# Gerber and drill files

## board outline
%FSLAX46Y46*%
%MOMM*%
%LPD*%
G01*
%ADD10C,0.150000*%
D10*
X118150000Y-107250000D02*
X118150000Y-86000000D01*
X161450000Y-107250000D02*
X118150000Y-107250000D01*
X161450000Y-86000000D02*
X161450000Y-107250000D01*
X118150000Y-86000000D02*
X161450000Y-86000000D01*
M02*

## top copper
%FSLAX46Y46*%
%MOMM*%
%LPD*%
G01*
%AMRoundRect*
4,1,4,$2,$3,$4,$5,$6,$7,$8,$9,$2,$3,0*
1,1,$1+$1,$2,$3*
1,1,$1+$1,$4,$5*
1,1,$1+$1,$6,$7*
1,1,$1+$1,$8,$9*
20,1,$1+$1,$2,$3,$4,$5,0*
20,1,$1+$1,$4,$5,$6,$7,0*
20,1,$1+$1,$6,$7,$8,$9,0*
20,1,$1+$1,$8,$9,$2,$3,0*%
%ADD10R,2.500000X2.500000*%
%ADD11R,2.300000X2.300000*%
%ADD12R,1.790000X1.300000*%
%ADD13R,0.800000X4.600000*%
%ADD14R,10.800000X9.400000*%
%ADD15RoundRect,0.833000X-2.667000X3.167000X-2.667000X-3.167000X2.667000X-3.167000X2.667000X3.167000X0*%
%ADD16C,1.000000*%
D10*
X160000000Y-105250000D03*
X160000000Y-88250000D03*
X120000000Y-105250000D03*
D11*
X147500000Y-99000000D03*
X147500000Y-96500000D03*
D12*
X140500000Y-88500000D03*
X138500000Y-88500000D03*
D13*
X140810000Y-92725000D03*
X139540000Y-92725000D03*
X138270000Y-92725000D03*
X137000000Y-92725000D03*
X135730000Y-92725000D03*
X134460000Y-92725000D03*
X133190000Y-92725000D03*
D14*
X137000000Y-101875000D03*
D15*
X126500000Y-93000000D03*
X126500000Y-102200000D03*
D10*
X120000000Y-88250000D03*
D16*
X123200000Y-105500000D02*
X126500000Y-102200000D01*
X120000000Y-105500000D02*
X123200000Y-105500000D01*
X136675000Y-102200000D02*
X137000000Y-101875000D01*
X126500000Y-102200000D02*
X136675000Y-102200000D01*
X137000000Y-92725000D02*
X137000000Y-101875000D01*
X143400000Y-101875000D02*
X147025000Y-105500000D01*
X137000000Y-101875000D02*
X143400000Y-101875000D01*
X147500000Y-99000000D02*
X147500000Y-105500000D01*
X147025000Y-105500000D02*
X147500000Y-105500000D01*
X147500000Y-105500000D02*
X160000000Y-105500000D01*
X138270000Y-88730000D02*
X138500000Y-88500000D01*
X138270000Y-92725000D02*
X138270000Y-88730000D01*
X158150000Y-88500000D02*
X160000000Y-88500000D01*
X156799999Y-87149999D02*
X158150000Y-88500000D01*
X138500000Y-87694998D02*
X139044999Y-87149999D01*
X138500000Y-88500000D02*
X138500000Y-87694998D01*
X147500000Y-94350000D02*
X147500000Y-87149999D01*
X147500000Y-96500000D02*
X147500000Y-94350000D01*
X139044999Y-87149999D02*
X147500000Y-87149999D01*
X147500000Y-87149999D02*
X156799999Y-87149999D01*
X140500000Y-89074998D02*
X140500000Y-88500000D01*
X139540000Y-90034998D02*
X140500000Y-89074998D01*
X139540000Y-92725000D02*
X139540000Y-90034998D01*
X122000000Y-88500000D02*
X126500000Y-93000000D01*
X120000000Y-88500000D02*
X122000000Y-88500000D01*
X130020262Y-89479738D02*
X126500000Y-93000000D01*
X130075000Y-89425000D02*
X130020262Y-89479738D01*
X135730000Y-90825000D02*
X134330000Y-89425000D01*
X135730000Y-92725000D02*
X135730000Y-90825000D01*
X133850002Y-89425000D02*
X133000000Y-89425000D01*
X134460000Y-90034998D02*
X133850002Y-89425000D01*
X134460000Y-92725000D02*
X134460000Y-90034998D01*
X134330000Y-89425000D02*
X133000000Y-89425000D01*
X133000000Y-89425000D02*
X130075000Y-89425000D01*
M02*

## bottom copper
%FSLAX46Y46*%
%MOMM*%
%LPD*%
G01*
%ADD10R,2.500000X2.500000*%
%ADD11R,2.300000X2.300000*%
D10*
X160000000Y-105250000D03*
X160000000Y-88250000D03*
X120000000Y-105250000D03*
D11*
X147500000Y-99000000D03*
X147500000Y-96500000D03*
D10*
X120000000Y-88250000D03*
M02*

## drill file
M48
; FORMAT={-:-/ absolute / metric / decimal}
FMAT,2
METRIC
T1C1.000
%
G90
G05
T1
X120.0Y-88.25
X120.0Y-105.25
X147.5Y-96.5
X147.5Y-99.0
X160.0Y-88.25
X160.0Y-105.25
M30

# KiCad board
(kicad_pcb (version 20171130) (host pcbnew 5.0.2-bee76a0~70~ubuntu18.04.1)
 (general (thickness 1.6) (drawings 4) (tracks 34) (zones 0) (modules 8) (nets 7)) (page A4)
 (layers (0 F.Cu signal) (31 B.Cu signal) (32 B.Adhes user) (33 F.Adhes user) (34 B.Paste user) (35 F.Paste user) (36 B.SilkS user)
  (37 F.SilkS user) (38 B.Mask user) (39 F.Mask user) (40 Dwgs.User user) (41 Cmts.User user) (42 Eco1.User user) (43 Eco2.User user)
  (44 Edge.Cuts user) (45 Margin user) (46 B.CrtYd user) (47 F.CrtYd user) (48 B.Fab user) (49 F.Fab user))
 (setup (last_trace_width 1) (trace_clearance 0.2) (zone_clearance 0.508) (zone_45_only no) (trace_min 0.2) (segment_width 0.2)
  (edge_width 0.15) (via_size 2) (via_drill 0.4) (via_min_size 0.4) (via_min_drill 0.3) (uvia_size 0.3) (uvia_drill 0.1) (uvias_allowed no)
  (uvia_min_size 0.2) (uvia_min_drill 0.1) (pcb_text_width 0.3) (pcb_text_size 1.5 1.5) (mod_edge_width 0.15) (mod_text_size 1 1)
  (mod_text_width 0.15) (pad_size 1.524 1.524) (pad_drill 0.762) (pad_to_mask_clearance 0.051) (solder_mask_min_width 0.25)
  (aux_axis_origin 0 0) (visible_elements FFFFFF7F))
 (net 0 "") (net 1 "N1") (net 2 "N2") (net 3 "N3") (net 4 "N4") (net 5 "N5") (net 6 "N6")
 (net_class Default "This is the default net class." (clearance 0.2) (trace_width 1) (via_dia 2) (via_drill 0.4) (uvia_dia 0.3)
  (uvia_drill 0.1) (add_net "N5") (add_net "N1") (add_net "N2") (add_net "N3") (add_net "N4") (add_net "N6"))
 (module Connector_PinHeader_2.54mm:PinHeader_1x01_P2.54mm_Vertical (layer F.Cu) (at 160 105.25)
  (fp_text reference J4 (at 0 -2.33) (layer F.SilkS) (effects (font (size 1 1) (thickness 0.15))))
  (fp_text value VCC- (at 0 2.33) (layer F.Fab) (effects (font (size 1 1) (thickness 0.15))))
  (pad 1 thru_hole rect (at 0 0) (size 2.5 2.5) (drill 1) (layers *.Cu *.Mask) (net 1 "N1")))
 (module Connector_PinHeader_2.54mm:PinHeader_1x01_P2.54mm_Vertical (layer F.Cu) (at 160 88.25)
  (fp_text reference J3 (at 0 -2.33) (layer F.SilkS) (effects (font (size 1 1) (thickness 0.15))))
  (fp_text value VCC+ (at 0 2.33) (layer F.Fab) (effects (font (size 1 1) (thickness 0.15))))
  (pad 1 thru_hole rect (at 0 0) (size 2.5 2.5) (drill 1) (layers *.Cu *.Mask) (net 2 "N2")))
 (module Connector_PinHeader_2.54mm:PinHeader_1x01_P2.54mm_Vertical (layer F.Cu) (at 120 105.25)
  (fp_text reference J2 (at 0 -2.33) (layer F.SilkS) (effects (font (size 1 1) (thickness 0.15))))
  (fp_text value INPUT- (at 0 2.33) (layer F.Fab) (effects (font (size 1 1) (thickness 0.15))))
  (pad 1 thru_hole rect (at 0 0) (size 2.5 2.5) (drill 1) (layers *.Cu *.Mask) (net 1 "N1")))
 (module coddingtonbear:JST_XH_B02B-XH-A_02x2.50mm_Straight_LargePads (layer F.Cu) (at 147.5 96.5 270)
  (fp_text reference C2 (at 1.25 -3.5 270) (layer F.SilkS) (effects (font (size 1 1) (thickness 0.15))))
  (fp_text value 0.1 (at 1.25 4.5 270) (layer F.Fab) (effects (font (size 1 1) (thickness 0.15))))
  (pad 2 thru_hole rect (at 2.5 0 270) (size 2.3 2.3) (drill 1) (layers *.Cu *.Mask) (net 1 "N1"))
  (pad 1 thru_hole rect (at 0 0 270) (size 2.3 2.3) (drill 1) (layers *.Cu *.Mask) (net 2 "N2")))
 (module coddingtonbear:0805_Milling (layer F.Cu) (at 139.5 88.5)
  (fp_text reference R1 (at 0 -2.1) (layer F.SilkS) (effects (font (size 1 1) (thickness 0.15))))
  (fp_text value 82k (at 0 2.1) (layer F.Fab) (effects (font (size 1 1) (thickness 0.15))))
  (pad 2 smd rect (at 1 0) (size 1.79 1.3) (layers F.Cu F.Paste F.Mask) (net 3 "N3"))
  (pad 1 smd rect (at -1 0) (size 1.79 1.3) (layers F.Cu F.Paste F.Mask) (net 2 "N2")))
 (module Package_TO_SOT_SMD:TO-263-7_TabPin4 (layer F.Cu) (at 137 98.5 270)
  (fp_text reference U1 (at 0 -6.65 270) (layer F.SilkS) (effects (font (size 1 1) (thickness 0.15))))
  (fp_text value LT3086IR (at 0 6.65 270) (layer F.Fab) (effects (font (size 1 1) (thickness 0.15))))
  (pad 1 smd rect (at -5.775 -3.81 270) (size 4.6 0.8) (layers F.Cu F.Paste F.Mask) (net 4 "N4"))
  (pad 2 smd rect (at -5.775 -2.54 270) (size 4.6 0.8) (layers F.Cu F.Paste F.Mask) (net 3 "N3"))
  (pad 3 smd rect (at -5.775 -1.27 270) (size 4.6 0.8) (layers F.Cu F.Paste F.Mask) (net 2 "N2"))
  (pad 4 smd rect (at -5.775 0 270) (size 4.6 0.8) (layers F.Cu F.Paste F.Mask) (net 1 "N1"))
  (pad 5 smd rect (at -5.775 1.27 270) (size 4.6 0.8) (layers F.Cu F.Paste F.Mask) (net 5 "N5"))
  (pad 6 smd rect (at -5.775 2.54 270) (size 4.6 0.8) (layers F.Cu F.Paste F.Mask) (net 5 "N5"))
  (pad 7 smd rect (at -5.775 3.81 270) (size 4.6 0.8) (layers F.Cu F.Paste F.Mask) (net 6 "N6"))
  (pad 4 smd rect (at 3.375 0 270) (size 9.4 10.8) (layers F.Cu F.Mask) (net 1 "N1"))
  (pad "" smd rect (at 5.8 2.775 270) (size 4.55 5.25) (layers F.Paste))
  (pad "" smd rect (at 0.95 -2.775 270) (size 4.55 5.25) (layers F.Paste))
  (pad "" smd rect (at 5.8 -2.775 270) (size 4.55 5.25) (layers F.Paste))
  (pad "" smd rect (at 0.95 2.775 270) (size 4.55 5.25) (layers F.Paste)))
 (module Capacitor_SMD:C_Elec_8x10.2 (layer F.Cu) (at 126.5 97.6 270)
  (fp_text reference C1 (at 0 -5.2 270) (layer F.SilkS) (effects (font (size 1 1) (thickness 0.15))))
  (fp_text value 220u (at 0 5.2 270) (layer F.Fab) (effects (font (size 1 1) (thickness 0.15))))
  (pad 1 smd roundrect (at -4.6 0 270) (size 8 7) (layers F.Cu F.Paste F.Mask) (roundrect_rratio 0.119) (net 5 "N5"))
  (pad 2 smd roundrect (at 4.6 0 270) (size 8 7) (layers F.Cu F.Paste F.Mask) (roundrect_rratio 0.119) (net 1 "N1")))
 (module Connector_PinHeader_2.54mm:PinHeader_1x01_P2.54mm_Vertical (layer F.Cu) (at 120 88.25)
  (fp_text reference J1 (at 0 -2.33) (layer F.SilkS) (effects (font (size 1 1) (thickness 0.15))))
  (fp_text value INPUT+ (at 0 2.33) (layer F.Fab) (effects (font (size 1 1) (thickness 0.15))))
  (pad 1 thru_hole rect (at 0 0) (size 2.5 2.5) (drill 1) (layers *.Cu *.Mask) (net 5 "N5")))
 (gr_line (start 118.15 107.25) (end 118.15 86) (layer Edge.Cuts) (width 0.15))
 (gr_line (start 161.45 107.25) (end 118.15 107.25) (layer Edge.Cuts) (width 0.15))
 (gr_line (start 161.45 86) (end 161.45 107.25) (layer Edge.Cuts) (width 0.15))
 (gr_line (start 118.15 86) (end 161.45 86) (layer Edge.Cuts) (width 0.15))
 (segment (start 123.2 105.5) (end 126.5 102.2) (width 1) (layer F.Cu) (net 1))
 (segment (start 120 105.5) (end 123.2 105.5) (width 1) (layer F.Cu) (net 1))
 (segment (start 136.675 102.2) (end 137 101.875) (width 1) (layer F.Cu) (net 1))
 (segment (start 126.5 102.2) (end 136.675 102.2) (width 1) (layer F.Cu) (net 1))
 (segment (start 137 92.725) (end 137 101.875) (width 1) (layer F.Cu) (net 1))
 (segment (start 143.4 101.875) (end 147.025 105.5) (width 1) (layer F.Cu) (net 1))
 (segment (start 137 101.875) (end 143.4 101.875) (width 1) (layer F.Cu) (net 1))
 (segment (start 147.5 99) (end 147.5 105.5) (width 1) (layer F.Cu) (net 1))
 (segment (start 147.025 105.5) (end 147.5 105.5) (width 1) (layer F.Cu) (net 1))
 (segment (start 147.5 105.5) (end 160 105.5) (width 1) (layer F.Cu) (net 1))
 (segment (start 138.27 88.73) (end 138.5 88.5) (width 1) (layer F.Cu) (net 2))
 (segment (start 138.27 92.725) (end 138.27 88.73) (width 1) (layer F.Cu) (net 2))
 (segment (start 158.15 88.5) (end 160 88.5) (width 1) (layer F.Cu) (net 2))
 (segment (start 156.799999 87.149999) (end 158.15 88.5) (width 1) (layer F.Cu) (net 2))
 (segment (start 138.5 87.694998) (end 139.044999 87.149999) (width 1) (layer F.Cu) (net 2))
 (segment (start 138.5 88.5) (end 138.5 87.694998) (width 1) (layer F.Cu) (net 2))
 (segment (start 147.5 94.35) (end 147.5 87.149999) (width 1) (layer F.Cu) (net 2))
 (segment (start 147.5 96.5) (end 147.5 94.35) (width 1) (layer F.Cu) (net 2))
 (segment (start 139.044999 87.149999) (end 147.5 87.149999) (width 1) (layer F.Cu) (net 2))
 (segment (start 147.5 87.149999) (end 156.799999 87.149999) (width 1) (layer F.Cu) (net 2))
 (segment (start 140.5 89.074998) (end 140.5 88.5) (width 1) (layer F.Cu) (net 3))
 (segment (start 139.54 90.034998) (end 140.5 89.074998) (width 1) (layer F.Cu) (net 3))
 (segment (start 139.54 92.725) (end 139.54 90.034998) (width 1) (layer F.Cu) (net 3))
 (segment (start 122 88.5) (end 126.5 93) (width 1) (layer F.Cu) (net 5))
 (segment (start 120 88.5) (end 122 88.5) (width 1) (layer F.Cu) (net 5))
 (segment (start 130.020262 89.479738) (end 126.5 93) (width 1) (layer F.Cu) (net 5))
 (segment (start 130.075 89.425) (end 130.020262 89.479738) (width 1) (layer F.Cu) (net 5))
 (segment (start 135.73 90.825) (end 134.33 89.425) (width 1) (layer F.Cu) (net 5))
 (segment (start 135.73 92.725) (end 135.73 90.825) (width 1) (layer F.Cu) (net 5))
 (segment (start 133.850002 89.425) (end 133 89.425) (width 1) (layer F.Cu) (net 5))
 (segment (start 134.46 90.034998) (end 133.850002 89.425) (width 1) (layer F.Cu) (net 5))
 (segment (start 134.46 92.725) (end 134.46 90.034998) (width 1) (layer F.Cu) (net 5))
 (segment (start 134.33 89.425) (end 133 89.425) (width 1) (layer F.Cu) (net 5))
 (segment (start 133 89.425) (end 130.075 89.425) (width 1) (layer F.Cu) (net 5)))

